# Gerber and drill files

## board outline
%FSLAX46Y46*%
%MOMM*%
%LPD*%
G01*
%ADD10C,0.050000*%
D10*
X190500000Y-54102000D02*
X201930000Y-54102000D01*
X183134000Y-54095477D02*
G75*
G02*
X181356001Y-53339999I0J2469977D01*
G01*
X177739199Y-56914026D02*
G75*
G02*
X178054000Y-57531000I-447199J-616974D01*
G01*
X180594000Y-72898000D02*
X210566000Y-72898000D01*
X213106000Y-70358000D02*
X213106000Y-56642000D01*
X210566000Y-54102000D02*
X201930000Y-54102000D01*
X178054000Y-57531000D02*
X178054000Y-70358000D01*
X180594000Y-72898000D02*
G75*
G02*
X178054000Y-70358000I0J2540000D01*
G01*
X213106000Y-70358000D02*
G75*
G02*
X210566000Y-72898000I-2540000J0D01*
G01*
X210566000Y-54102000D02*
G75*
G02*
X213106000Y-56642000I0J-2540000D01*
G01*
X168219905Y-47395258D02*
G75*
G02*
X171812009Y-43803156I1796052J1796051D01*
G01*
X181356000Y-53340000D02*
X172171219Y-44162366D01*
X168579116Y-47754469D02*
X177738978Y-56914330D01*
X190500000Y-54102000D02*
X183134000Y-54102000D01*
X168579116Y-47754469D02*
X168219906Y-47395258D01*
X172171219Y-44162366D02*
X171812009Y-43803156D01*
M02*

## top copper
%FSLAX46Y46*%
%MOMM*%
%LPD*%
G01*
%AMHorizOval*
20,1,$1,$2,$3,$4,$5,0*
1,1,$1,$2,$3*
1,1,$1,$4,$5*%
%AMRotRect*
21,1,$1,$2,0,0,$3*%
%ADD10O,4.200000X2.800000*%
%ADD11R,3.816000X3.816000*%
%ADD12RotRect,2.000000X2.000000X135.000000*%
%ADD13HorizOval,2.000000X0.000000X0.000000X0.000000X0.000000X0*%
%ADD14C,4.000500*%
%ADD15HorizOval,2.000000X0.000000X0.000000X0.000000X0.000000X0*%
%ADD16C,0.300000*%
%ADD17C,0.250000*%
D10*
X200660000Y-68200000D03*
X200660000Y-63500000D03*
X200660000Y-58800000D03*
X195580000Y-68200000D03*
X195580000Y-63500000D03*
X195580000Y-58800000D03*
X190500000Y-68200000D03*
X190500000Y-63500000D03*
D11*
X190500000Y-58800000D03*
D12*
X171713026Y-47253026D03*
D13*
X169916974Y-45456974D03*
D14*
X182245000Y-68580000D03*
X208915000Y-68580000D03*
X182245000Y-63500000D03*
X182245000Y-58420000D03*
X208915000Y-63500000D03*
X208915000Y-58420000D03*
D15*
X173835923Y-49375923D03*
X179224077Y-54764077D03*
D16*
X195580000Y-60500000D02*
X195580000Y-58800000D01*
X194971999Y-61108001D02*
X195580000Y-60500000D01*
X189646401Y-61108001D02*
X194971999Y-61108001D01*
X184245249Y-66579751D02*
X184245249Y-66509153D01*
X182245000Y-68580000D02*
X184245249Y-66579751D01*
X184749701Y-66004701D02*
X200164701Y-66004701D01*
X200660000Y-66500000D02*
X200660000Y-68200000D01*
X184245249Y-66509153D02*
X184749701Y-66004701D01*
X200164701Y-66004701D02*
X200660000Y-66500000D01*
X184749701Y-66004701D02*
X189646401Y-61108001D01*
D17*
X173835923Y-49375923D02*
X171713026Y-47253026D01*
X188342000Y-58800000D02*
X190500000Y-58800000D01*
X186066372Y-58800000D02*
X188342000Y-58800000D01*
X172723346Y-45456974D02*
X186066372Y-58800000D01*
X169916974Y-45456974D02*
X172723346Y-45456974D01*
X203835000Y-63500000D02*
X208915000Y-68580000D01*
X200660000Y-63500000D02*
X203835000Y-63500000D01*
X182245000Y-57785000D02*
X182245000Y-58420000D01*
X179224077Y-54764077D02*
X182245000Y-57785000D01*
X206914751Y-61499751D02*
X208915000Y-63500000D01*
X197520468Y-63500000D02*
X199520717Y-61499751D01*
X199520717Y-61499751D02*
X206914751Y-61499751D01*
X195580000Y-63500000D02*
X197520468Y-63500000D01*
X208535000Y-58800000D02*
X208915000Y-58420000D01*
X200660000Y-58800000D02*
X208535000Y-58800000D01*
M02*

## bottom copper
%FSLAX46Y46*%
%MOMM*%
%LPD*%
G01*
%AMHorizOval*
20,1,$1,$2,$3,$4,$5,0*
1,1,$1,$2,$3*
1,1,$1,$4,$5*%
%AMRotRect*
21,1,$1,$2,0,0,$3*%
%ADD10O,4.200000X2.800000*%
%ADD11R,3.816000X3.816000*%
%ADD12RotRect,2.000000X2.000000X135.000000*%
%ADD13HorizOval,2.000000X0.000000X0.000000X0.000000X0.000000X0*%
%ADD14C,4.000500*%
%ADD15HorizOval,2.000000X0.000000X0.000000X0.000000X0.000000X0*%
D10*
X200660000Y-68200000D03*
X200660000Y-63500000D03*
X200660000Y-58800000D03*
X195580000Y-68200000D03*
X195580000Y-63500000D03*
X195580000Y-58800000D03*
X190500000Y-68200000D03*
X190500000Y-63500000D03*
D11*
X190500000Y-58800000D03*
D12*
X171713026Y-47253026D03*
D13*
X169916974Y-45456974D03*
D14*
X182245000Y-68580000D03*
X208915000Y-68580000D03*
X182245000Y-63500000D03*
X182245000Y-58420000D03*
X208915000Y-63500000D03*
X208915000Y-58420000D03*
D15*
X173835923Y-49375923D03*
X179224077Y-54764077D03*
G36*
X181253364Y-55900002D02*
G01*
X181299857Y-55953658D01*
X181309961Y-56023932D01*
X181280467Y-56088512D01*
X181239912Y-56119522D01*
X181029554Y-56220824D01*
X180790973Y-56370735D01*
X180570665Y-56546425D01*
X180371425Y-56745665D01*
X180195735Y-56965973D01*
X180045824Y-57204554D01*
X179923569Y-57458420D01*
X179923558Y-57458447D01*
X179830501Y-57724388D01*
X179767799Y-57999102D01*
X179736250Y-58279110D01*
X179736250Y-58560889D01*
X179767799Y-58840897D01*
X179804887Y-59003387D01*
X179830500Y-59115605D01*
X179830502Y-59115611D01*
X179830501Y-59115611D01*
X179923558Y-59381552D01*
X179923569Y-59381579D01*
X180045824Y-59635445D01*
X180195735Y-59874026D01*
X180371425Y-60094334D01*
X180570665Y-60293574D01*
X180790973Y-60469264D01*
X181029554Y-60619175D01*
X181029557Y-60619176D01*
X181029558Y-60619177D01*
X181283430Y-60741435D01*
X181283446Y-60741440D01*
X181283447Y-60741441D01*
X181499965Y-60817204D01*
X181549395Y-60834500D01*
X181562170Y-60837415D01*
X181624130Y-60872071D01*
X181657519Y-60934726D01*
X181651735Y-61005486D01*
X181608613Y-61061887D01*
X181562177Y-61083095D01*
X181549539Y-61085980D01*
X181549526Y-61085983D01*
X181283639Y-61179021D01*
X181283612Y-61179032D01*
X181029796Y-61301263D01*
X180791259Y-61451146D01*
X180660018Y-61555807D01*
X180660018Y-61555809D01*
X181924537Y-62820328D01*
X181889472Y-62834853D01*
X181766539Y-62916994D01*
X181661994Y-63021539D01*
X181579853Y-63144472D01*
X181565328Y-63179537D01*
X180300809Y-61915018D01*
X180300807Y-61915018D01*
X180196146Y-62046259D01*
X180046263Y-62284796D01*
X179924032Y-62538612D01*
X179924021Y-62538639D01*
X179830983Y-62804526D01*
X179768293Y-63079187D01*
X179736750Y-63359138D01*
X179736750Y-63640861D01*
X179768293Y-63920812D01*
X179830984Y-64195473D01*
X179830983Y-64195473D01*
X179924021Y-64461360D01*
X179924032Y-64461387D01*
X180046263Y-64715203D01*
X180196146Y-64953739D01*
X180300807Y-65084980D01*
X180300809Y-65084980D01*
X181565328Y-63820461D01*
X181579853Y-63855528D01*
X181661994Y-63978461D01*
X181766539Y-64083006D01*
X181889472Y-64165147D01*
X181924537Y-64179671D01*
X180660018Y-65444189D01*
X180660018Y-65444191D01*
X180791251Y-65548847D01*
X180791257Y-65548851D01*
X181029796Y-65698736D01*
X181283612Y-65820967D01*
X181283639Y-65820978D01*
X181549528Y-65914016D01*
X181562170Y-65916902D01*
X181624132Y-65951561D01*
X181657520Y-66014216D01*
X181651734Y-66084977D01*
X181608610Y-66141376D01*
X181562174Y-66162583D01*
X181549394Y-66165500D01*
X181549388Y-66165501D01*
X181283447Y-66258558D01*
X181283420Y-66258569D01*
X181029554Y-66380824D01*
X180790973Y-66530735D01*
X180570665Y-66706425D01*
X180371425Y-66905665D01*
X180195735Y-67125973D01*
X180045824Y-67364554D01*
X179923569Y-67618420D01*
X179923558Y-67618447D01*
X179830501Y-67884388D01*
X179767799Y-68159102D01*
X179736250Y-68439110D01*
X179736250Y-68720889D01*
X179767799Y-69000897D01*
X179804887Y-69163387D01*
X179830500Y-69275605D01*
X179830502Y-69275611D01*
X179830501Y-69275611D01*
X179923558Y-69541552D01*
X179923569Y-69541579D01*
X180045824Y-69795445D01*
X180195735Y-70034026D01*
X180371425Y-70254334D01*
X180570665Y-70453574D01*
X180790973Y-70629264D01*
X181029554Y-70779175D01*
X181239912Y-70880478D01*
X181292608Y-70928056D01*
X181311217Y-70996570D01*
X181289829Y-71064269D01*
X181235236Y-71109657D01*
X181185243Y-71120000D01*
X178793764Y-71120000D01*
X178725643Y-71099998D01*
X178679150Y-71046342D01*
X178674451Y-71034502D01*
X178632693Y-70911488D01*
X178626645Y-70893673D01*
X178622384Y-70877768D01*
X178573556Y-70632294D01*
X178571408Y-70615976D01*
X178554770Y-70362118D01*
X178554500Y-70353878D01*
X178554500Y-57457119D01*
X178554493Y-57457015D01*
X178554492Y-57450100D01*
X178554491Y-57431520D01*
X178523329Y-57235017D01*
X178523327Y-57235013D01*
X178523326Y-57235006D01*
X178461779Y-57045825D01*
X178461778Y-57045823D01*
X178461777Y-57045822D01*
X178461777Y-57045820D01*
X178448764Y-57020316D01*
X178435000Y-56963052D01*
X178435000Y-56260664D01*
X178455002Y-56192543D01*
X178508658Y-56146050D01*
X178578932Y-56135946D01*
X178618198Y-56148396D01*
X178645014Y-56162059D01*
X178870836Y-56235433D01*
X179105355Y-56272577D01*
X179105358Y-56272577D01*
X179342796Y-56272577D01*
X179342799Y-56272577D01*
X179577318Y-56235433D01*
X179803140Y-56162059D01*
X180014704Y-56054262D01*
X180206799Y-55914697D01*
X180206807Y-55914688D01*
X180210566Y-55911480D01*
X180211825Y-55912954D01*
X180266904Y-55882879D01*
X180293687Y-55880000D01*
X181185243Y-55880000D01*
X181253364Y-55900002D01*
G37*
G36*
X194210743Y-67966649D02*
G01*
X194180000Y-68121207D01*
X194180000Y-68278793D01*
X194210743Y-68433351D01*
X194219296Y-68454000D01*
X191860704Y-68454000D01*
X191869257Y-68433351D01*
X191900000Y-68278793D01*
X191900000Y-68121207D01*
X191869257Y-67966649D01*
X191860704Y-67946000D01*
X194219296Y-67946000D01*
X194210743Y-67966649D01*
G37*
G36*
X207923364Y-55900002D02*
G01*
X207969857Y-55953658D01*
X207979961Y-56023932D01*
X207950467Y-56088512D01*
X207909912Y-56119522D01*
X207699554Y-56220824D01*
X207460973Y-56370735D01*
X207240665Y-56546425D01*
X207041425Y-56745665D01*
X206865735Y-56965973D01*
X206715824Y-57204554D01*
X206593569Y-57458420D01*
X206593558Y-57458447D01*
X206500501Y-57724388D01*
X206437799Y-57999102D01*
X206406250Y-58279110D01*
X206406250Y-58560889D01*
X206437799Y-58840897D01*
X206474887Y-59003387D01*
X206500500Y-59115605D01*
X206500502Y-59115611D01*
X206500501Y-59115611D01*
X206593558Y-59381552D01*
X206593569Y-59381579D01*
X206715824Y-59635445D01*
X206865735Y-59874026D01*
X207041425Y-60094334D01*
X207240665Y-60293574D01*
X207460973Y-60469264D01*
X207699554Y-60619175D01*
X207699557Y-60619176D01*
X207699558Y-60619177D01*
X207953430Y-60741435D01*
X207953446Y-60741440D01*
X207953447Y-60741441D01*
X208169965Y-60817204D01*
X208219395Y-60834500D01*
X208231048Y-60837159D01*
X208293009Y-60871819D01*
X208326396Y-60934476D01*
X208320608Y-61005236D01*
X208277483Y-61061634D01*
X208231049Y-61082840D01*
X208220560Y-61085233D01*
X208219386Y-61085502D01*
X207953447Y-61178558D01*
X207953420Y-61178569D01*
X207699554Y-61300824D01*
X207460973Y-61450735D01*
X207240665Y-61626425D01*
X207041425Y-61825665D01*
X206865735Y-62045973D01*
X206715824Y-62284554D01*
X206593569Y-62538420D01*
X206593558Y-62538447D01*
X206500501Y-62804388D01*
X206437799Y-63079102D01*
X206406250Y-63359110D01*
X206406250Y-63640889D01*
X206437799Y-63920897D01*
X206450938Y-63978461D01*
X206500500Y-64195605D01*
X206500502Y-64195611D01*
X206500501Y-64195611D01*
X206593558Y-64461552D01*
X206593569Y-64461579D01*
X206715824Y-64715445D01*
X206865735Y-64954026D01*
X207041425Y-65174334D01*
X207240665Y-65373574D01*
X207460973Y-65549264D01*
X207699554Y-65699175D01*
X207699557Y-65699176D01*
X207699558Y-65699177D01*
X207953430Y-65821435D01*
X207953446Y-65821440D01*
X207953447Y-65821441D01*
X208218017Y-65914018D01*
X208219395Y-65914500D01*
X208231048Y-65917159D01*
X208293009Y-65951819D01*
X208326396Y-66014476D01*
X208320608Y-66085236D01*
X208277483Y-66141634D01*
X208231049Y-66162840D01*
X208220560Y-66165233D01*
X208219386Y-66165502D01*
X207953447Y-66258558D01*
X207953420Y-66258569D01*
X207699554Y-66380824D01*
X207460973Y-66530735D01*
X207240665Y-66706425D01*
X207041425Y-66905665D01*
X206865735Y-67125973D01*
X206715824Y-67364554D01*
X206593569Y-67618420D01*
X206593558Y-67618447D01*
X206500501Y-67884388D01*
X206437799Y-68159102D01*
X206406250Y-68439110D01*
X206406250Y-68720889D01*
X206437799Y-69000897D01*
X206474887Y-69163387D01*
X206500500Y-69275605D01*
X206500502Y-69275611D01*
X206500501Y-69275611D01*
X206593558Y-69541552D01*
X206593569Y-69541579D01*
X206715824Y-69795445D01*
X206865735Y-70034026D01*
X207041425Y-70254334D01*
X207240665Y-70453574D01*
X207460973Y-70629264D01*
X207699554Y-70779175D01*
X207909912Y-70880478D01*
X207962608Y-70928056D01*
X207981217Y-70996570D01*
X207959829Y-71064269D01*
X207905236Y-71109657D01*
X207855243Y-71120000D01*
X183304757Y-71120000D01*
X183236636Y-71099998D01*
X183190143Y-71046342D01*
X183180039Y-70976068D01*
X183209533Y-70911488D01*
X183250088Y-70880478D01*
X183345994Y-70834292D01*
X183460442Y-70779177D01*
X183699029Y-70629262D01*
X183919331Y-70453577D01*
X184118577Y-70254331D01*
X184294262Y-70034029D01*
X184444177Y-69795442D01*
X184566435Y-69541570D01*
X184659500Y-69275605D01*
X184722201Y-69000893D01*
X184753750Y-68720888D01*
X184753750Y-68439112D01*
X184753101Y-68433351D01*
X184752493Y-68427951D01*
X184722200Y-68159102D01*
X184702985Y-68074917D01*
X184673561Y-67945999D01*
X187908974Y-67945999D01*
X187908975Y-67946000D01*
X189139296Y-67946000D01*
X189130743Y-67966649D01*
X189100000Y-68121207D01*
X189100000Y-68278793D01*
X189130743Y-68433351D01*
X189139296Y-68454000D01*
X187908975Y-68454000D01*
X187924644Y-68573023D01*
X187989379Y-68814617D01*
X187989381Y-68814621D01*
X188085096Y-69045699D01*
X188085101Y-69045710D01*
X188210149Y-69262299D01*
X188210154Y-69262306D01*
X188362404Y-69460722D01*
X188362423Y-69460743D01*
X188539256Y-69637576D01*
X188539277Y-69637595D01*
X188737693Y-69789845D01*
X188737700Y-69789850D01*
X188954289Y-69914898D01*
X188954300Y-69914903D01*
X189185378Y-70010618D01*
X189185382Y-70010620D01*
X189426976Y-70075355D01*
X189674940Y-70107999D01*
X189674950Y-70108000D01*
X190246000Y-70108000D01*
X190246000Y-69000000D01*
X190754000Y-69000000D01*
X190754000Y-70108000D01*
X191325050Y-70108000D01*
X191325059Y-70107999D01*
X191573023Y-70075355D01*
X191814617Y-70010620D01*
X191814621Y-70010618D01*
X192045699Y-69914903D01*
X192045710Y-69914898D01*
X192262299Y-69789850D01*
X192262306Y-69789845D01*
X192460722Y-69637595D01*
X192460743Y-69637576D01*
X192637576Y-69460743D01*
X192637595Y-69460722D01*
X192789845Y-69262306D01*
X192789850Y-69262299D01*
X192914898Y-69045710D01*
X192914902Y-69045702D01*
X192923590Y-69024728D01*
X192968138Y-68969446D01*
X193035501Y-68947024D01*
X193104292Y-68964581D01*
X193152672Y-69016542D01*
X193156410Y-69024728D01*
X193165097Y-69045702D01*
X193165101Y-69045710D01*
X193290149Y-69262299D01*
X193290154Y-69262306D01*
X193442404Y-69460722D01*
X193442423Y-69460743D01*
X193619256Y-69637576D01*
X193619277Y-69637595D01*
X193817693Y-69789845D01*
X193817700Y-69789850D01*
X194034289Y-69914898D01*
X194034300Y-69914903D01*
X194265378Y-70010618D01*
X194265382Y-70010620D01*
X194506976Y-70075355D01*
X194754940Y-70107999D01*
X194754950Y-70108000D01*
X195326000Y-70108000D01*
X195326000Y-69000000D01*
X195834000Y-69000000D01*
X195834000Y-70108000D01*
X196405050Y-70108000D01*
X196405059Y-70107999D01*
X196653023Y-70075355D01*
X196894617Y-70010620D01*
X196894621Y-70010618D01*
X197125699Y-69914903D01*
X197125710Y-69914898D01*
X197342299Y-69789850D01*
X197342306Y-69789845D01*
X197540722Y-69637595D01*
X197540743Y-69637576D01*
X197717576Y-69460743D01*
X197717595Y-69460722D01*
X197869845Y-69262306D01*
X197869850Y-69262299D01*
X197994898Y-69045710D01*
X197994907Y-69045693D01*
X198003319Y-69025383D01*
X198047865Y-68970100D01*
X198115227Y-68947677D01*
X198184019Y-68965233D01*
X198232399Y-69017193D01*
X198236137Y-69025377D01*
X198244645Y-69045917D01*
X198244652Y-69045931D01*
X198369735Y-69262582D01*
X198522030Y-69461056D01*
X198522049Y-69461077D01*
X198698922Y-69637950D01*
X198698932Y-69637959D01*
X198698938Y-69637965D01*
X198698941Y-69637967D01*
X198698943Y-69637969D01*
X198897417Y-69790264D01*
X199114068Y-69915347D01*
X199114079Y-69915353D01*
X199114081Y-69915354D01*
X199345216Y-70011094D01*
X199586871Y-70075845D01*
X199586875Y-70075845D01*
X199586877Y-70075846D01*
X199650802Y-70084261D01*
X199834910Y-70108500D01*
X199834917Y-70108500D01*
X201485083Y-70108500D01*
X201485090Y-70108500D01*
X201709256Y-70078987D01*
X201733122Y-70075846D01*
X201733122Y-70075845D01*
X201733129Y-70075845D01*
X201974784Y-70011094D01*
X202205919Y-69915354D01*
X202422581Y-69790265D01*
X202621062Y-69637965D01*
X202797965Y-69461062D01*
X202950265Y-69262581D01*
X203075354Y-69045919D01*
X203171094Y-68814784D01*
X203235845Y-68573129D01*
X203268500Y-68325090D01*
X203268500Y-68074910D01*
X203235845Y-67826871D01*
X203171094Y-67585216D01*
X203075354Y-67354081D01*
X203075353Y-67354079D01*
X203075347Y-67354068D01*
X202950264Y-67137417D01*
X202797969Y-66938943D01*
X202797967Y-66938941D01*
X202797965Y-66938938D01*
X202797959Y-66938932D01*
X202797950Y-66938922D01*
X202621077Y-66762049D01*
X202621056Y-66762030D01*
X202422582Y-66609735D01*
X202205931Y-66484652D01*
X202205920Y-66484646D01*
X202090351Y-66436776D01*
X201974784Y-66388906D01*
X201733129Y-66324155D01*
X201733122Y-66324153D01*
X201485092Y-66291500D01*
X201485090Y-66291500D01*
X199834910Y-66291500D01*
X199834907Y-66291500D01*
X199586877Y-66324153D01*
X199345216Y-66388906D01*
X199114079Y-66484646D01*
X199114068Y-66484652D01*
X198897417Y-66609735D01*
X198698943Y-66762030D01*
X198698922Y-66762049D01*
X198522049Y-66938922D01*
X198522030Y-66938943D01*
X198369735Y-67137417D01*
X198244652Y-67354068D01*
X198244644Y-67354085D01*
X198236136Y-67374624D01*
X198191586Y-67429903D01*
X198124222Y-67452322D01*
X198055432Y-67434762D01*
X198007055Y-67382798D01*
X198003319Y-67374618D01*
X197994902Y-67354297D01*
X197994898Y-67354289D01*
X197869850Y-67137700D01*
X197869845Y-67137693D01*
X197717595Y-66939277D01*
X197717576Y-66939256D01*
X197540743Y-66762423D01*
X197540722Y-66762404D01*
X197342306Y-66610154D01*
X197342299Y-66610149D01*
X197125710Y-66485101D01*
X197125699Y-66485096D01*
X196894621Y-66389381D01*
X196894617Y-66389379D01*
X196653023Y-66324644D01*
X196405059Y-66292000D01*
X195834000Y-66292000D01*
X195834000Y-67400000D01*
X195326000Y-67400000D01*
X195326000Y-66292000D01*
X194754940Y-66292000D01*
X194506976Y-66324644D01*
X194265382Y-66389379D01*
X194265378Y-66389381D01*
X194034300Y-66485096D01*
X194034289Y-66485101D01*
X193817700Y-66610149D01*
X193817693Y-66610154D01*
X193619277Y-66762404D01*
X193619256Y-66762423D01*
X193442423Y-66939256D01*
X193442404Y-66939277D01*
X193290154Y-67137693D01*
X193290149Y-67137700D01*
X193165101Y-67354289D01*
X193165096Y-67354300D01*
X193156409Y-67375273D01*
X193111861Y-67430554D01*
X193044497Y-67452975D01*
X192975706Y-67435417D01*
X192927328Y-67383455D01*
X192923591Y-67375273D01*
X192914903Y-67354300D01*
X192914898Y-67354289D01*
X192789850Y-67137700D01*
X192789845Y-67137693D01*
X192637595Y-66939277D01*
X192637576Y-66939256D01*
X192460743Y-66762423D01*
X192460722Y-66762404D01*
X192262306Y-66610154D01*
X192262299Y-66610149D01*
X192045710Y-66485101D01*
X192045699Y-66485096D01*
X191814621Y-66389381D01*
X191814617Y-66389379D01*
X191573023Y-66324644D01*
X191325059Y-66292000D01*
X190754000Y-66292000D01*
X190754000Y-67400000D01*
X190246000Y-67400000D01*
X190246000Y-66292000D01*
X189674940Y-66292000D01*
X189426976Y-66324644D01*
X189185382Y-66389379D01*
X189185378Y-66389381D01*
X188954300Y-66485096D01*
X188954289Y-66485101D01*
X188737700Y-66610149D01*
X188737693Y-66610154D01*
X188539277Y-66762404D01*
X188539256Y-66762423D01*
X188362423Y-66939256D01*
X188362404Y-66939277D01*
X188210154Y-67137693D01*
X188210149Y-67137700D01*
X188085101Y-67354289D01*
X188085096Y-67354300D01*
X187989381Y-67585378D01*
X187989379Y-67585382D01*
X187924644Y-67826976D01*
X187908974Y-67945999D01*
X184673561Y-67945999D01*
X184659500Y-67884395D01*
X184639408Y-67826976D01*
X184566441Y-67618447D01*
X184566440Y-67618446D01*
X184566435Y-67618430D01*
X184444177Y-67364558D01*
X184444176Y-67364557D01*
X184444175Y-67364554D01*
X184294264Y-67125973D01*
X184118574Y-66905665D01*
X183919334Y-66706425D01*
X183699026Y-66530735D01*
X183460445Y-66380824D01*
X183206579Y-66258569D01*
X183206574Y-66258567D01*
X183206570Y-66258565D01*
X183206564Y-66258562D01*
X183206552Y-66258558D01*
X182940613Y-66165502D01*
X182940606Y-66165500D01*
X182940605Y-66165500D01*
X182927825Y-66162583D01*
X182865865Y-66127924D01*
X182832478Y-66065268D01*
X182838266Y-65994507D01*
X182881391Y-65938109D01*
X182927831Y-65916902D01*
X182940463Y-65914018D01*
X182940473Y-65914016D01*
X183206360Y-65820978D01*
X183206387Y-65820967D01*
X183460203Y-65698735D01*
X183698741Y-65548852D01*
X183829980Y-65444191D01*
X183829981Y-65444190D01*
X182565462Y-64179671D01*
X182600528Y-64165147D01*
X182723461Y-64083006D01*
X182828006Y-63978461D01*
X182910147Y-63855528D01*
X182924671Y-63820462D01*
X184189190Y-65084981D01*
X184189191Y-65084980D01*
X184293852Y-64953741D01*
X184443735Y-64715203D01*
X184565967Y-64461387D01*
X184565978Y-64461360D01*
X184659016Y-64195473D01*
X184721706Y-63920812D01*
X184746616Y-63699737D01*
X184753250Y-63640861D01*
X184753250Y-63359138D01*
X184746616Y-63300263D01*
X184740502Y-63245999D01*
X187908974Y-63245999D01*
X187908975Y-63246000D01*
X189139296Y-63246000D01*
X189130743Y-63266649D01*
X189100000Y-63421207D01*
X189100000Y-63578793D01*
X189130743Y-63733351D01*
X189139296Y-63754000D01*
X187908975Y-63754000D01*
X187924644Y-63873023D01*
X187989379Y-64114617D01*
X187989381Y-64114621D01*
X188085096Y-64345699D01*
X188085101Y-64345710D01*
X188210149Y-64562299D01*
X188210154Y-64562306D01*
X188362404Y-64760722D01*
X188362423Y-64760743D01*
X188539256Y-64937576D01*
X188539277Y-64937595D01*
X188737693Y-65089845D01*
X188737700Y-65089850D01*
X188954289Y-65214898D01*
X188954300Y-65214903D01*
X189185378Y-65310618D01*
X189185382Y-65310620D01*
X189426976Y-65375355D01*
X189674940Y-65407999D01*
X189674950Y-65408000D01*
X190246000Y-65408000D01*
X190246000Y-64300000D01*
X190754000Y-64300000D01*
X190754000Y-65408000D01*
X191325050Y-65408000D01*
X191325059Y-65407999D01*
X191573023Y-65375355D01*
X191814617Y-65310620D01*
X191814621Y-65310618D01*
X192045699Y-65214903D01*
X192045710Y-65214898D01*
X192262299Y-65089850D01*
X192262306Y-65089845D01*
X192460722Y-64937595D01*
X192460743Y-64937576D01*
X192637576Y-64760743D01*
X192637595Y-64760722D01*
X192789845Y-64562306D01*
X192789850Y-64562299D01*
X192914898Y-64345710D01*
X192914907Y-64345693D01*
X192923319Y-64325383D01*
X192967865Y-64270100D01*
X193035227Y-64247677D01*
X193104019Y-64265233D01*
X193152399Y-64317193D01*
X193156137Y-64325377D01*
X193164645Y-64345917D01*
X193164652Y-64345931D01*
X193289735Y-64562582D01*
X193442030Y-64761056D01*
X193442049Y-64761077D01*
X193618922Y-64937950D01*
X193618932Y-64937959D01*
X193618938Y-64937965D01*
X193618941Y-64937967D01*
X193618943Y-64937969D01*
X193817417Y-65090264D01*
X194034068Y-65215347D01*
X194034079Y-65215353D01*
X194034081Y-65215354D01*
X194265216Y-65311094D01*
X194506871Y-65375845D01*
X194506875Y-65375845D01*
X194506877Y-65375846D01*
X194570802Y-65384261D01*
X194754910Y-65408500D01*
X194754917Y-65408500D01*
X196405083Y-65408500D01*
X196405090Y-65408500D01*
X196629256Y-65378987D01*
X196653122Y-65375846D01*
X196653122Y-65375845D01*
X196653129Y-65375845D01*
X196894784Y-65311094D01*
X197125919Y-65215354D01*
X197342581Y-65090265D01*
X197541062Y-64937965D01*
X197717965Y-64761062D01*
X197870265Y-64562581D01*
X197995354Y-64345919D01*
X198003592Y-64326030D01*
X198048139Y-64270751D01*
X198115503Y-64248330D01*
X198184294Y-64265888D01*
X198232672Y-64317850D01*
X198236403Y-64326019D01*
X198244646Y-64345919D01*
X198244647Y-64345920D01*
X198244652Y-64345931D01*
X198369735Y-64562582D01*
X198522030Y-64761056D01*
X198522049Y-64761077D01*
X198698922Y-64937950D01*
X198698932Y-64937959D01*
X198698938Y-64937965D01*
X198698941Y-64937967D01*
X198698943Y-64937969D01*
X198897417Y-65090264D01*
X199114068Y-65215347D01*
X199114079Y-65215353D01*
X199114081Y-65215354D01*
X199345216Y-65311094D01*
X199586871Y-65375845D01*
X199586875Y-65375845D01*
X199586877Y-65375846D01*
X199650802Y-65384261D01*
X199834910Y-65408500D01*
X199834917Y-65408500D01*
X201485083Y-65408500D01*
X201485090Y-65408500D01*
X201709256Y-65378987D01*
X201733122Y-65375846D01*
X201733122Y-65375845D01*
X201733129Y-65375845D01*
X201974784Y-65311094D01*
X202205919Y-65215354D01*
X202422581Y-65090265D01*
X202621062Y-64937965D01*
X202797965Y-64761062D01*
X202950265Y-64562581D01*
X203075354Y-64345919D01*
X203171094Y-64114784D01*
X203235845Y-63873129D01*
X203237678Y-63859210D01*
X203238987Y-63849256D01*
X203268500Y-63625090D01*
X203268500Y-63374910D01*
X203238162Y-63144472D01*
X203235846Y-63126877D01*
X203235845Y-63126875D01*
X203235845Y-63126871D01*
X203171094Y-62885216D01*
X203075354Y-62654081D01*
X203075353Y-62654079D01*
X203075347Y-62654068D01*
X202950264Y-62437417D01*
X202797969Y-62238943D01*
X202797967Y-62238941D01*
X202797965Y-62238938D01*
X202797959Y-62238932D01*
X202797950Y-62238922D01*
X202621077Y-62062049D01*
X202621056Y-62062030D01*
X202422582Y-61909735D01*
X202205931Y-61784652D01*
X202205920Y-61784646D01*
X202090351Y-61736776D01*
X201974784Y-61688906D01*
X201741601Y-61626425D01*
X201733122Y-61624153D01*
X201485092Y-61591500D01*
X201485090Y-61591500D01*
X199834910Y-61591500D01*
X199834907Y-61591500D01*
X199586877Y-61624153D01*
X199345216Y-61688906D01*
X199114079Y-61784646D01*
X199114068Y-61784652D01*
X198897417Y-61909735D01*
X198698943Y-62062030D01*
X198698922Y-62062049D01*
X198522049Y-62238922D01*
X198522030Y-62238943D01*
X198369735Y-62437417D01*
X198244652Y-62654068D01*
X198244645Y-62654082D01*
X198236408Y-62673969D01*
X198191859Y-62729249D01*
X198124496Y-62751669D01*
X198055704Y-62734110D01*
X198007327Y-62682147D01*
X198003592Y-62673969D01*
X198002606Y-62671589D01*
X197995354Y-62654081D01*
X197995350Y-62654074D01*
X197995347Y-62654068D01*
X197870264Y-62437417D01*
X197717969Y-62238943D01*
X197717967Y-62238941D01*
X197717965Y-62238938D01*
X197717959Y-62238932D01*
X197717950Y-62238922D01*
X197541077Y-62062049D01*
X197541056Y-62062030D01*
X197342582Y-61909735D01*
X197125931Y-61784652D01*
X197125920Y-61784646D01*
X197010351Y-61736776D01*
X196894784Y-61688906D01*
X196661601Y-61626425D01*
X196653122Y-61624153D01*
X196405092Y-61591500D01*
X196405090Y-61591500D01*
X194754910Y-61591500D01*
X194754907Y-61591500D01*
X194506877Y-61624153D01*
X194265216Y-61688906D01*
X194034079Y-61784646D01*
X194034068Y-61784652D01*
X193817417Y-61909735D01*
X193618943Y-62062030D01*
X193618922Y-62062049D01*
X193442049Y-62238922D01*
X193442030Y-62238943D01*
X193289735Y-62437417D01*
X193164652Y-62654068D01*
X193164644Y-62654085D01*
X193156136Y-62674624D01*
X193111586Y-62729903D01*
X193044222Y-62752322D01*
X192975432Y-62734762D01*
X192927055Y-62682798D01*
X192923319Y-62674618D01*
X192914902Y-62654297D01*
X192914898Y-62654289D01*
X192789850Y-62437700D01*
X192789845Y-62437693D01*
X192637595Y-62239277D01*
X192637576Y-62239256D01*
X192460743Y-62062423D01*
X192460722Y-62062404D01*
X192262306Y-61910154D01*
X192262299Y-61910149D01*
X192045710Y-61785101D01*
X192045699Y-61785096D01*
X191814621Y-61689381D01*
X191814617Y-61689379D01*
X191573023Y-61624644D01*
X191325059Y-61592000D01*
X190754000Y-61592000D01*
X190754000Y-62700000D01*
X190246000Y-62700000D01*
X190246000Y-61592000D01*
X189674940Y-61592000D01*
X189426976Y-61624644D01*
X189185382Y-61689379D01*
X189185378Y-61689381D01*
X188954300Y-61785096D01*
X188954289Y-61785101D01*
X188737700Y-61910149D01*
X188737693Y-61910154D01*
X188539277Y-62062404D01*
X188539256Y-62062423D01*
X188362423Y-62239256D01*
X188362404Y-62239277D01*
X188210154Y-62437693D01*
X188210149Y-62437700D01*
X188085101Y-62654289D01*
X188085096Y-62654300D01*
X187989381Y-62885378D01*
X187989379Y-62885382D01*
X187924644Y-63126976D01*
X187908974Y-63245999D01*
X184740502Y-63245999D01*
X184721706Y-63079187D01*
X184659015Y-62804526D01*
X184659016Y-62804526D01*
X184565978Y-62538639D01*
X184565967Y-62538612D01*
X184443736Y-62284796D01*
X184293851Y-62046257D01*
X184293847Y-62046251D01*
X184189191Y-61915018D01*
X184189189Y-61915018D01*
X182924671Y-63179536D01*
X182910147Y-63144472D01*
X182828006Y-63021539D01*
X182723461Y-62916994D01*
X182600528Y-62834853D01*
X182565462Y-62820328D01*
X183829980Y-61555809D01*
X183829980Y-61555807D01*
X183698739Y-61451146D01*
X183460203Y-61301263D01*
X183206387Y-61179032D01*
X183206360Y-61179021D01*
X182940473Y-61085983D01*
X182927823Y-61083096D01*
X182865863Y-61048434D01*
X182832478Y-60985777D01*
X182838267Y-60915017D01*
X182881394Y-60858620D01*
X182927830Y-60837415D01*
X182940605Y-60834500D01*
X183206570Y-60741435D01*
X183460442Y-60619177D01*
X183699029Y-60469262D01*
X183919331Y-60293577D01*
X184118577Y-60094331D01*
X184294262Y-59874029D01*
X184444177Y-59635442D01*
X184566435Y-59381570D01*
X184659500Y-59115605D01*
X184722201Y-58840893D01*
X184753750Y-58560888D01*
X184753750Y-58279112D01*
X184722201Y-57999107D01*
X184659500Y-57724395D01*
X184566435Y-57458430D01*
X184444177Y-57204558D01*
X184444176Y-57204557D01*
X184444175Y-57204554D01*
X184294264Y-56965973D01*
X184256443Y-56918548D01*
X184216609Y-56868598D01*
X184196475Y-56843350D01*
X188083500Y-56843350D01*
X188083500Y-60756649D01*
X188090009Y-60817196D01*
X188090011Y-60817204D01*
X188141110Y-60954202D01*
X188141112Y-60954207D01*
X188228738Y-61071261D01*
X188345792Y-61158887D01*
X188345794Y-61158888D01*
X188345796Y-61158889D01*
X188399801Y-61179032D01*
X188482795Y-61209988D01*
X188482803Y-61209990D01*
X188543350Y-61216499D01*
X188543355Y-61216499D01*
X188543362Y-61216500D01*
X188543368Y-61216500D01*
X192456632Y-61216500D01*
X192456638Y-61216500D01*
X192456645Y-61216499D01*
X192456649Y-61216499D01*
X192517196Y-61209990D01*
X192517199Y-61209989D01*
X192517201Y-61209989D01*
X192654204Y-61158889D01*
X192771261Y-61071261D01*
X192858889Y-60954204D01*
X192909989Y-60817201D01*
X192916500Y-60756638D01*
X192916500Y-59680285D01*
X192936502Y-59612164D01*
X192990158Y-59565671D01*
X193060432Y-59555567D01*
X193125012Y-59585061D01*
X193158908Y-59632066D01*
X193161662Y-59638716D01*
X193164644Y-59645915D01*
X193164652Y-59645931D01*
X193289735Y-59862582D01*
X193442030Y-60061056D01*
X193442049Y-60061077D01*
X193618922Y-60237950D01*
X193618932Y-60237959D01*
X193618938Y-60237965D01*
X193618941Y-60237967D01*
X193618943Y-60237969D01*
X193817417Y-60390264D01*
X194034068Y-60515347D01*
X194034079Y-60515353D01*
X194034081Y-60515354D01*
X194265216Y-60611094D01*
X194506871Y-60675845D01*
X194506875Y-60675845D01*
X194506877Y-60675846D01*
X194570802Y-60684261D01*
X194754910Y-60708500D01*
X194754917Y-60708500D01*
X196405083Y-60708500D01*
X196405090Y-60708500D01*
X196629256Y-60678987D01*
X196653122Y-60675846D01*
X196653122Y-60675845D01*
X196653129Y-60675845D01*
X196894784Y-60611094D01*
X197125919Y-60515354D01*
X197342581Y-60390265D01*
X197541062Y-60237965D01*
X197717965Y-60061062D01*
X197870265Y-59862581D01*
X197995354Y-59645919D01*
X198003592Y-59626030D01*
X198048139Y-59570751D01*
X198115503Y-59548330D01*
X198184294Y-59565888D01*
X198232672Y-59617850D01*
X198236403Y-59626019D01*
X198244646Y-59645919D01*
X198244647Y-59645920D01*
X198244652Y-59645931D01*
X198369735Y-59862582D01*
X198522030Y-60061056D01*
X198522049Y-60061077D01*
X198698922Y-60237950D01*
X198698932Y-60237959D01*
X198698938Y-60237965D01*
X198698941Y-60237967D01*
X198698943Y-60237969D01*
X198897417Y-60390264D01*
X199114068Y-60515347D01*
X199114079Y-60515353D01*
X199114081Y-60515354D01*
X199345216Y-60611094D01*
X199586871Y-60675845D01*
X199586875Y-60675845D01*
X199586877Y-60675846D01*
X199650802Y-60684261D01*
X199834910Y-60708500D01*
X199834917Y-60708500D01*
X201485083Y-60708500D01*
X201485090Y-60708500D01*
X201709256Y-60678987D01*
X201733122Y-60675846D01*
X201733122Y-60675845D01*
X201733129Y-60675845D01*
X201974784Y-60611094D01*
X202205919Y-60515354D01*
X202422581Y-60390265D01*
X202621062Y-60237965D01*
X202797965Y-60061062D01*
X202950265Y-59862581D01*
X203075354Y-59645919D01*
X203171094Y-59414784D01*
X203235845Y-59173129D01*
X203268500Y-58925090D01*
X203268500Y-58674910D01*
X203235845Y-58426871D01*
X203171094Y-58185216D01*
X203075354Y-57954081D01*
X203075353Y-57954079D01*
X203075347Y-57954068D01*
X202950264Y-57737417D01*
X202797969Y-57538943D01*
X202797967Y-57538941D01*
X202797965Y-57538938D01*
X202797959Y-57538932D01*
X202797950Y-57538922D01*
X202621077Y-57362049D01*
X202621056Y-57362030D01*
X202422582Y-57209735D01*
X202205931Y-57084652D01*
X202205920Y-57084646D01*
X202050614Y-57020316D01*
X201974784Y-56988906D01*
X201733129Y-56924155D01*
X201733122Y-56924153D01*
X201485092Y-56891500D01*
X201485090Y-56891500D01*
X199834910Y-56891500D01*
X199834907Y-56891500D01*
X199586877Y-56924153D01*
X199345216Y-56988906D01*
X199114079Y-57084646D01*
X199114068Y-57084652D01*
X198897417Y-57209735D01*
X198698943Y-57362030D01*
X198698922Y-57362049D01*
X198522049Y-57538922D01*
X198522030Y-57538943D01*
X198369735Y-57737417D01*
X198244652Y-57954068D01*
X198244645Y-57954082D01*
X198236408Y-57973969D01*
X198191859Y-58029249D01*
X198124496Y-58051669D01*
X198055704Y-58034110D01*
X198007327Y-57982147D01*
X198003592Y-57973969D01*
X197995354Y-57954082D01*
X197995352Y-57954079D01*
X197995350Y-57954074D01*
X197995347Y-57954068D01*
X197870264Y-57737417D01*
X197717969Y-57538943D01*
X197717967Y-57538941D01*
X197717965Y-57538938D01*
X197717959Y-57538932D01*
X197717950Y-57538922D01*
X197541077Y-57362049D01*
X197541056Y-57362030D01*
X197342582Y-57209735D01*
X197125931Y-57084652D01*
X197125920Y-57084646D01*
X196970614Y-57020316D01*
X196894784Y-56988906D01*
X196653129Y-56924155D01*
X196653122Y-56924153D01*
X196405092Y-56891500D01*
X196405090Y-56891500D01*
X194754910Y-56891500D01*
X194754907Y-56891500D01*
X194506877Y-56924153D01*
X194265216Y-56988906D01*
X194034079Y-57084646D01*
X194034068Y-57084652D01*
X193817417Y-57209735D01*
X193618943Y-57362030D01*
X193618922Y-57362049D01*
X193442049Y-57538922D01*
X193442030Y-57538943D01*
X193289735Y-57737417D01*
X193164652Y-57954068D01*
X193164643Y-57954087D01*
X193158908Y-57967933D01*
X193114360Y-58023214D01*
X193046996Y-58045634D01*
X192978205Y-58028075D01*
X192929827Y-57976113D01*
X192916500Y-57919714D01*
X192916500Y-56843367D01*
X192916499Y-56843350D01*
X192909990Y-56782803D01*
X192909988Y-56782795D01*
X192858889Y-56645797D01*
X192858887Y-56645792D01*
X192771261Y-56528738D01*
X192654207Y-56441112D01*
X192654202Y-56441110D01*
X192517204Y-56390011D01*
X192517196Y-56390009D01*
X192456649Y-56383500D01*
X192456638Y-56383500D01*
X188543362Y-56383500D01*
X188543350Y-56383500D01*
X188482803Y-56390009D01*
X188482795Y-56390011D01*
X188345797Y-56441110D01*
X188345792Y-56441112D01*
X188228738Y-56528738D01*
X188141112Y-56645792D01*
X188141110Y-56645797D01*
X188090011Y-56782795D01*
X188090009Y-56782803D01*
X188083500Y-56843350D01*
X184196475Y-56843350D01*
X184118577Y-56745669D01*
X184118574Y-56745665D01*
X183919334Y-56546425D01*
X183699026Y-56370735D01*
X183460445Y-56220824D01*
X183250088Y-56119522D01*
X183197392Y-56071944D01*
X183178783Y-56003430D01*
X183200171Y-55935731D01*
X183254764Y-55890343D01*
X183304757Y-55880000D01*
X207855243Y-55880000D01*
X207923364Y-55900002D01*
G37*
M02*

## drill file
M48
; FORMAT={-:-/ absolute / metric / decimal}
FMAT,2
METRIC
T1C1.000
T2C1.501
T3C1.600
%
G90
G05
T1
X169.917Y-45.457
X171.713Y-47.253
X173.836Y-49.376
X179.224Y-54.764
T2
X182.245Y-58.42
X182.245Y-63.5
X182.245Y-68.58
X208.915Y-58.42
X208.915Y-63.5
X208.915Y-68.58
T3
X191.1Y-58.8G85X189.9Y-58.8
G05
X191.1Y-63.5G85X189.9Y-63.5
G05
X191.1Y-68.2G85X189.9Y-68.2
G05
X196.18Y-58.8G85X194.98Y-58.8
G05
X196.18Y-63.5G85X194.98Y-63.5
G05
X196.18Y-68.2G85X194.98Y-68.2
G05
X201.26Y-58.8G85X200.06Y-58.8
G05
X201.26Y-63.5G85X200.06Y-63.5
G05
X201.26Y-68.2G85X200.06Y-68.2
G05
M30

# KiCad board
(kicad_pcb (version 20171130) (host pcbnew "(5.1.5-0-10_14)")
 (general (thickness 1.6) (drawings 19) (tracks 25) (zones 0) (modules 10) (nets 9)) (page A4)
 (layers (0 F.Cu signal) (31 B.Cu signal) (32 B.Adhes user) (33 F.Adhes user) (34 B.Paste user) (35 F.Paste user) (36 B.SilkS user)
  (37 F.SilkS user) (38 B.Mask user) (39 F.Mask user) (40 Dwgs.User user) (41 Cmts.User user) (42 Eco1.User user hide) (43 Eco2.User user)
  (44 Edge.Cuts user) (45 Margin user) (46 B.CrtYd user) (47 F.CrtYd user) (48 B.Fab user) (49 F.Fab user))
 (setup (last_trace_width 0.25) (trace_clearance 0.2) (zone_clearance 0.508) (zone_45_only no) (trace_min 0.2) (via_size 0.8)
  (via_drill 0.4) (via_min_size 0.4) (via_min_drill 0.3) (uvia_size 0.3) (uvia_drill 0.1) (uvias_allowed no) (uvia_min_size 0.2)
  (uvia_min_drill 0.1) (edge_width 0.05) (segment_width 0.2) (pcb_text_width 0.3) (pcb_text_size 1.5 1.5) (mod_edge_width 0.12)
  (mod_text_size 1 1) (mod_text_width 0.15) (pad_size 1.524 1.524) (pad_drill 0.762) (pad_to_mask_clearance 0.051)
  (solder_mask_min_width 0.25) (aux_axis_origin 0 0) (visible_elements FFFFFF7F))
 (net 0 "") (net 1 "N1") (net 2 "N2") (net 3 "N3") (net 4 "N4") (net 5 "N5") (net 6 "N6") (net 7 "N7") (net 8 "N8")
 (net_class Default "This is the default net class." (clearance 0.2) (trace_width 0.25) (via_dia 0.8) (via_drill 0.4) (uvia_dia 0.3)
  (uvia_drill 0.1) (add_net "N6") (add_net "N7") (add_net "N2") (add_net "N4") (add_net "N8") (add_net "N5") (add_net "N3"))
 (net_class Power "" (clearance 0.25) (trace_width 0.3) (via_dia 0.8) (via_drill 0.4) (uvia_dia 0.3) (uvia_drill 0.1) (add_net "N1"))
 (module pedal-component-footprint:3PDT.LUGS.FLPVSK (layer F.Cu) (at 195.58 63.5)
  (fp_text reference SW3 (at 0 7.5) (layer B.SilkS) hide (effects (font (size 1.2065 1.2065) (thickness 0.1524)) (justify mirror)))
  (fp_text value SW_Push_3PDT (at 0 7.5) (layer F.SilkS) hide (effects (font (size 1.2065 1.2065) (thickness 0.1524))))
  (pad 9 thru_hole oval (at 5.08 4.7 180) (size 4.2 2.8) (drill oval 2.8 1.6) (layers *.Cu *.Mask) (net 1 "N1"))
  (pad 8 thru_hole oval (at 5.08 0 180) (size 4.2 2.8) (drill oval 2.8 1.6) (layers *.Cu *.Mask) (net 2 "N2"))
  (pad 7 thru_hole oval (at 5.08 -4.7 180) (size 4.2 2.8) (drill oval 2.8 1.6) (layers *.Cu *.Mask) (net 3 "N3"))
  (pad 6 thru_hole oval (at 0 4.7 180) (size 4.2 2.8) (drill oval 2.8 1.6) (layers *.Cu *.Mask) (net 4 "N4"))
  (pad 5 thru_hole oval (at 0 0 180) (size 4.2 2.8) (drill oval 2.8 1.6) (layers *.Cu *.Mask) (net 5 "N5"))
  (pad 4 thru_hole oval (at 0 -4.7 180) (size 4.2 2.8) (drill oval 2.8 1.6) (layers *.Cu *.Mask) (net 1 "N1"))
  (pad 3 thru_hole oval (at -5.08 4.7 180) (size 4.2 2.8) (drill oval 2.8 1.6) (layers *.Cu *.Mask) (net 4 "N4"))
  (pad 2 thru_hole oval (at -5.08 0 180) (size 4.2 2.8) (drill oval 2.8 1.6) (layers *.Cu *.Mask) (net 4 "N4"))
  (pad 1 thru_hole rect (at -5.08 -4.7 180) (size 3.816 3.816) (drill oval 2.8 1.6) (layers *.Cu *.Mask) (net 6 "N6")))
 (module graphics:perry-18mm (layer F.Cu) (at 195.58 62.23)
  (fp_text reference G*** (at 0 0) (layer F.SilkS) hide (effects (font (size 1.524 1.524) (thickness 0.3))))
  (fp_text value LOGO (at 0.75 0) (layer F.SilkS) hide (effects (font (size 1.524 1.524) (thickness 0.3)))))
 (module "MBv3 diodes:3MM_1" (layer F.Cu) (at 170.815 46.355 135)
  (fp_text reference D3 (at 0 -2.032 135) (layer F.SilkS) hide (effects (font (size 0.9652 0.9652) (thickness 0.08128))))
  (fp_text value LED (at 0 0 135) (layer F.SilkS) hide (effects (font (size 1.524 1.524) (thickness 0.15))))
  (pad 2 thru_hole rect (at -1.27 0 135) (size 2 2) (drill 1) (layers *.Cu *.Mask) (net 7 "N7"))
  (pad 1 thru_hole oval (at 1.27 0 135) (size 2 2) (drill 1) (layers *.Cu *.Mask) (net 6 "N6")))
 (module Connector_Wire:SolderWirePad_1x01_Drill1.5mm (layer F.Cu) (at 182.245 68.58 270)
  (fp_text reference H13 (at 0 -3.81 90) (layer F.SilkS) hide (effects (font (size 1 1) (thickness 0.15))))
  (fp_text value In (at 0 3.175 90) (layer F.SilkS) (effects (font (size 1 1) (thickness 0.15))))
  (pad 1 thru_hole circle (at 0 0 270) (size 4.0005 4.0005) (drill 1.50114) (layers *.Cu *.Mask) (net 1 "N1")))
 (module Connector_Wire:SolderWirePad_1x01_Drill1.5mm (layer F.Cu) (at 208.915 68.58 90)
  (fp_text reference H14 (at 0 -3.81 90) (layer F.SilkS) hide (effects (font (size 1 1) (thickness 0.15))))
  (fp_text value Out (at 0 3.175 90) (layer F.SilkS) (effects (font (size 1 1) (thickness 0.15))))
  (pad 1 thru_hole circle (at 0 0 90) (size 4.0005 4.0005) (drill 1.50114) (layers *.Cu *.Mask) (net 2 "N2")))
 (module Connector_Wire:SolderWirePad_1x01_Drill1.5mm (layer F.Cu) (at 182.245 63.5 270)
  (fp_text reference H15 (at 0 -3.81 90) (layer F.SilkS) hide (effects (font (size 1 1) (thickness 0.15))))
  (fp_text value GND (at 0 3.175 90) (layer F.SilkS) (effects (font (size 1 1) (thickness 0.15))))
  (pad 1 thru_hole circle (at 0 0 270) (size 4.0005 4.0005) (drill 1.50114) (layers *.Cu *.Mask) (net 4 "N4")))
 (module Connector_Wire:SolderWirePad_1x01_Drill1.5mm (layer F.Cu) (at 182.245 58.42 270)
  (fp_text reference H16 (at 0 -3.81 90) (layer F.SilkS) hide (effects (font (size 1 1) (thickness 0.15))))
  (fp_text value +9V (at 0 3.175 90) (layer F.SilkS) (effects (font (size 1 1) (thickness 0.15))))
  (pad 1 thru_hole circle (at 0 0 270) (size 4.0005 4.0005) (drill 1.50114) (layers *.Cu *.Mask) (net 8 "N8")))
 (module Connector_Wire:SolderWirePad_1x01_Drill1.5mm (layer F.Cu) (at 208.915 63.5 90)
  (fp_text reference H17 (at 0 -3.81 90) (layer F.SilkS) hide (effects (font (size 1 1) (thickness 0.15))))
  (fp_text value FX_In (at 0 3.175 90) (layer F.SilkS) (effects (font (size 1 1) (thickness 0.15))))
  (pad 1 thru_hole circle (at 0 0 90) (size 4.0005 4.0005) (drill 1.50114) (layers *.Cu *.Mask) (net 5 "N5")))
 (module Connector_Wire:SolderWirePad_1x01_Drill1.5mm (layer F.Cu) (at 208.915 58.42 90)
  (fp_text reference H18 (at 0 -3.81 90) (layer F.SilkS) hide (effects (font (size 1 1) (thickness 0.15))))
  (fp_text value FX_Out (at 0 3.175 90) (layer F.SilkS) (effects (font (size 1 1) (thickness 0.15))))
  (pad 1 thru_hole circle (at 0 0 90) (size 4.0005 4.0005) (drill 1.50114) (layers *.Cu *.Mask) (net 3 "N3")))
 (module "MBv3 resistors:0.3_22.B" (layer F.Cu) (at 176.53 52.07 315)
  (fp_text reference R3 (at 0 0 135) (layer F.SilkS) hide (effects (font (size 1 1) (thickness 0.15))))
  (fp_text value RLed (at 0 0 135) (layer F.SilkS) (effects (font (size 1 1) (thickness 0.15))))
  (pad 1 thru_hole oval (at -3.81 0 315) (size 2 2) (drill 1) (layers *.Cu *.Mask) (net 7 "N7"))
  (pad 2 thru_hole oval (at 3.81 0 315) (size 2 2) (drill 1) (layers *.Cu *.Mask) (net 8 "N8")))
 (gr_line (start 190.5 54.102) (end 201.93 54.102) (layer Edge.Cuts) (width 0.05))
 (gr_arc (start 183.134 51.6255) (end 181.356001 53.339999) (angle -46.04162668) (layer Edge.Cuts) (width 0.05))
 (gr_arc (start 177.292 57.531) (end 178.054 57.531) (angle -54.06445072) (layer Edge.Cuts) (width 0.05))
 (gr_line (start 180.594 72.898) (end 210.566 72.898) (layer Edge.Cuts) (width 0.05))
 (gr_line (start 213.106 70.358) (end 213.106 56.642) (layer Edge.Cuts) (width 0.05))
 (gr_line (start 210.566 54.102) (end 201.93 54.102) (layer Edge.Cuts) (width 0.05))
 (gr_line (start 178.054 57.531) (end 178.054 70.358) (layer Edge.Cuts) (width 0.05))
 (gr_arc (start 180.594 70.358) (end 178.054 70.358) (angle -90) (layer Edge.Cuts) (width 0.05))
 (gr_arc (start 210.566 70.358) (end 210.566 72.898) (angle -90) (layer Edge.Cuts) (width 0.05))
 (gr_arc (start 210.566 56.642) (end 213.106 56.642) (angle -90) (layer Edge.Cuts) (width 0.05))
 (gr_arc (start 170.015957 45.599207) (end 171.812009 43.803156) (angle -180) (layer Edge.Cuts) (width 0.05))
 (gr_line (start 181.356 53.34) (end 172.171219 44.162366) (layer Edge.Cuts) (width 0.05))
 (gr_line (start 168.579116 47.754469) (end 177.738978 56.91433) (layer Edge.Cuts) (width 0.05))
 (gr_line (start 190.5 54.102) (end 183.134 54.102) (layer Edge.Cuts) (width 0.05))
 (gr_line (start 168.579116 47.754469) (end 168.219906 47.395258) (layer Edge.Cuts) (width 0.05))
 (gr_line (start 172.171219 44.162366) (end 171.812009 43.803156) (layer Edge.Cuts) (width 0.05))
 (segment (start 195.58 60.5) (end 195.58 58.8) (width 0.3) (layer F.Cu) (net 1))
 (segment (start 194.971999 61.108001) (end 195.58 60.5) (width 0.3) (layer F.Cu) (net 1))
 (segment (start 189.646401 61.108001) (end 194.971999 61.108001) (width 0.3) (layer F.Cu) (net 1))
 (segment (start 184.245249 66.579751) (end 184.245249 66.509153) (width 0.3) (layer F.Cu) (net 1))
 (segment (start 182.245 68.58) (end 184.245249 66.579751) (width 0.3) (layer F.Cu) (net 1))
 (segment (start 184.749701 66.004701) (end 200.164701 66.004701) (width 0.3) (layer F.Cu) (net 1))
 (segment (start 200.66 66.5) (end 200.66 68.2) (width 0.3) (layer F.Cu) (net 1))
 (segment (start 184.245249 66.509153) (end 184.749701 66.004701) (width 0.3) (layer F.Cu) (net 1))
 (segment (start 200.164701 66.004701) (end 200.66 66.5) (width 0.3) (layer F.Cu) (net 1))
 (segment (start 184.749701 66.004701) (end 189.646401 61.108001) (width 0.3) (layer F.Cu) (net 1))
 (segment (start 173.835923 49.375923) (end 171.713026 47.253026) (width 0.25) (layer F.Cu) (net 7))
 (segment (start 188.342 58.8) (end 190.5 58.8) (width 0.25) (layer F.Cu) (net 6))
 (segment (start 186.066372 58.8) (end 188.342 58.8) (width 0.25) (layer F.Cu) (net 6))
 (segment (start 172.723346 45.456974) (end 186.066372 58.8) (width 0.25) (layer F.Cu) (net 6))
 (segment (start 169.916974 45.456974) (end 172.723346 45.456974) (width 0.25) (layer F.Cu) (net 6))
 (segment (start 203.835 63.5) (end 208.915 68.58) (width 0.25) (layer F.Cu) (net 2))
 (segment (start 200.66 63.5) (end 203.835 63.5) (width 0.25) (layer F.Cu) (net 2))
 (segment (start 182.245 57.785) (end 182.245 58.42) (width 0.25) (layer F.Cu) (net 8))
 (segment (start 179.224077 54.764077) (end 182.245 57.785) (width 0.25) (layer F.Cu) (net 8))
 (segment (start 206.914751 61.499751) (end 208.915 63.5) (width 0.25) (layer F.Cu) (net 5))
 (segment (start 197.520468 63.5) (end 199.520717 61.499751) (width 0.25) (layer F.Cu) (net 5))
 (segment (start 199.520717 61.499751) (end 206.914751 61.499751) (width 0.25) (layer F.Cu) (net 5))
 (segment (start 195.58 63.5) (end 197.520468 63.5) (width 0.25) (layer F.Cu) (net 5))
 (segment (start 208.535 58.8) (end 208.915 58.42) (width 0.25) (layer F.Cu) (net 3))
 (segment (start 200.66 58.8) (end 208.535 58.8) (width 0.25) (layer F.Cu) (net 3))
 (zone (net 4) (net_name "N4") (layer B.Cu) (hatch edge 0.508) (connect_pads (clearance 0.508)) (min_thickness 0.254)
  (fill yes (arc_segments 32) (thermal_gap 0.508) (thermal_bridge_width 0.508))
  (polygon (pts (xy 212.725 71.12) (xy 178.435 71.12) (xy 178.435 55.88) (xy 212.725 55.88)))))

